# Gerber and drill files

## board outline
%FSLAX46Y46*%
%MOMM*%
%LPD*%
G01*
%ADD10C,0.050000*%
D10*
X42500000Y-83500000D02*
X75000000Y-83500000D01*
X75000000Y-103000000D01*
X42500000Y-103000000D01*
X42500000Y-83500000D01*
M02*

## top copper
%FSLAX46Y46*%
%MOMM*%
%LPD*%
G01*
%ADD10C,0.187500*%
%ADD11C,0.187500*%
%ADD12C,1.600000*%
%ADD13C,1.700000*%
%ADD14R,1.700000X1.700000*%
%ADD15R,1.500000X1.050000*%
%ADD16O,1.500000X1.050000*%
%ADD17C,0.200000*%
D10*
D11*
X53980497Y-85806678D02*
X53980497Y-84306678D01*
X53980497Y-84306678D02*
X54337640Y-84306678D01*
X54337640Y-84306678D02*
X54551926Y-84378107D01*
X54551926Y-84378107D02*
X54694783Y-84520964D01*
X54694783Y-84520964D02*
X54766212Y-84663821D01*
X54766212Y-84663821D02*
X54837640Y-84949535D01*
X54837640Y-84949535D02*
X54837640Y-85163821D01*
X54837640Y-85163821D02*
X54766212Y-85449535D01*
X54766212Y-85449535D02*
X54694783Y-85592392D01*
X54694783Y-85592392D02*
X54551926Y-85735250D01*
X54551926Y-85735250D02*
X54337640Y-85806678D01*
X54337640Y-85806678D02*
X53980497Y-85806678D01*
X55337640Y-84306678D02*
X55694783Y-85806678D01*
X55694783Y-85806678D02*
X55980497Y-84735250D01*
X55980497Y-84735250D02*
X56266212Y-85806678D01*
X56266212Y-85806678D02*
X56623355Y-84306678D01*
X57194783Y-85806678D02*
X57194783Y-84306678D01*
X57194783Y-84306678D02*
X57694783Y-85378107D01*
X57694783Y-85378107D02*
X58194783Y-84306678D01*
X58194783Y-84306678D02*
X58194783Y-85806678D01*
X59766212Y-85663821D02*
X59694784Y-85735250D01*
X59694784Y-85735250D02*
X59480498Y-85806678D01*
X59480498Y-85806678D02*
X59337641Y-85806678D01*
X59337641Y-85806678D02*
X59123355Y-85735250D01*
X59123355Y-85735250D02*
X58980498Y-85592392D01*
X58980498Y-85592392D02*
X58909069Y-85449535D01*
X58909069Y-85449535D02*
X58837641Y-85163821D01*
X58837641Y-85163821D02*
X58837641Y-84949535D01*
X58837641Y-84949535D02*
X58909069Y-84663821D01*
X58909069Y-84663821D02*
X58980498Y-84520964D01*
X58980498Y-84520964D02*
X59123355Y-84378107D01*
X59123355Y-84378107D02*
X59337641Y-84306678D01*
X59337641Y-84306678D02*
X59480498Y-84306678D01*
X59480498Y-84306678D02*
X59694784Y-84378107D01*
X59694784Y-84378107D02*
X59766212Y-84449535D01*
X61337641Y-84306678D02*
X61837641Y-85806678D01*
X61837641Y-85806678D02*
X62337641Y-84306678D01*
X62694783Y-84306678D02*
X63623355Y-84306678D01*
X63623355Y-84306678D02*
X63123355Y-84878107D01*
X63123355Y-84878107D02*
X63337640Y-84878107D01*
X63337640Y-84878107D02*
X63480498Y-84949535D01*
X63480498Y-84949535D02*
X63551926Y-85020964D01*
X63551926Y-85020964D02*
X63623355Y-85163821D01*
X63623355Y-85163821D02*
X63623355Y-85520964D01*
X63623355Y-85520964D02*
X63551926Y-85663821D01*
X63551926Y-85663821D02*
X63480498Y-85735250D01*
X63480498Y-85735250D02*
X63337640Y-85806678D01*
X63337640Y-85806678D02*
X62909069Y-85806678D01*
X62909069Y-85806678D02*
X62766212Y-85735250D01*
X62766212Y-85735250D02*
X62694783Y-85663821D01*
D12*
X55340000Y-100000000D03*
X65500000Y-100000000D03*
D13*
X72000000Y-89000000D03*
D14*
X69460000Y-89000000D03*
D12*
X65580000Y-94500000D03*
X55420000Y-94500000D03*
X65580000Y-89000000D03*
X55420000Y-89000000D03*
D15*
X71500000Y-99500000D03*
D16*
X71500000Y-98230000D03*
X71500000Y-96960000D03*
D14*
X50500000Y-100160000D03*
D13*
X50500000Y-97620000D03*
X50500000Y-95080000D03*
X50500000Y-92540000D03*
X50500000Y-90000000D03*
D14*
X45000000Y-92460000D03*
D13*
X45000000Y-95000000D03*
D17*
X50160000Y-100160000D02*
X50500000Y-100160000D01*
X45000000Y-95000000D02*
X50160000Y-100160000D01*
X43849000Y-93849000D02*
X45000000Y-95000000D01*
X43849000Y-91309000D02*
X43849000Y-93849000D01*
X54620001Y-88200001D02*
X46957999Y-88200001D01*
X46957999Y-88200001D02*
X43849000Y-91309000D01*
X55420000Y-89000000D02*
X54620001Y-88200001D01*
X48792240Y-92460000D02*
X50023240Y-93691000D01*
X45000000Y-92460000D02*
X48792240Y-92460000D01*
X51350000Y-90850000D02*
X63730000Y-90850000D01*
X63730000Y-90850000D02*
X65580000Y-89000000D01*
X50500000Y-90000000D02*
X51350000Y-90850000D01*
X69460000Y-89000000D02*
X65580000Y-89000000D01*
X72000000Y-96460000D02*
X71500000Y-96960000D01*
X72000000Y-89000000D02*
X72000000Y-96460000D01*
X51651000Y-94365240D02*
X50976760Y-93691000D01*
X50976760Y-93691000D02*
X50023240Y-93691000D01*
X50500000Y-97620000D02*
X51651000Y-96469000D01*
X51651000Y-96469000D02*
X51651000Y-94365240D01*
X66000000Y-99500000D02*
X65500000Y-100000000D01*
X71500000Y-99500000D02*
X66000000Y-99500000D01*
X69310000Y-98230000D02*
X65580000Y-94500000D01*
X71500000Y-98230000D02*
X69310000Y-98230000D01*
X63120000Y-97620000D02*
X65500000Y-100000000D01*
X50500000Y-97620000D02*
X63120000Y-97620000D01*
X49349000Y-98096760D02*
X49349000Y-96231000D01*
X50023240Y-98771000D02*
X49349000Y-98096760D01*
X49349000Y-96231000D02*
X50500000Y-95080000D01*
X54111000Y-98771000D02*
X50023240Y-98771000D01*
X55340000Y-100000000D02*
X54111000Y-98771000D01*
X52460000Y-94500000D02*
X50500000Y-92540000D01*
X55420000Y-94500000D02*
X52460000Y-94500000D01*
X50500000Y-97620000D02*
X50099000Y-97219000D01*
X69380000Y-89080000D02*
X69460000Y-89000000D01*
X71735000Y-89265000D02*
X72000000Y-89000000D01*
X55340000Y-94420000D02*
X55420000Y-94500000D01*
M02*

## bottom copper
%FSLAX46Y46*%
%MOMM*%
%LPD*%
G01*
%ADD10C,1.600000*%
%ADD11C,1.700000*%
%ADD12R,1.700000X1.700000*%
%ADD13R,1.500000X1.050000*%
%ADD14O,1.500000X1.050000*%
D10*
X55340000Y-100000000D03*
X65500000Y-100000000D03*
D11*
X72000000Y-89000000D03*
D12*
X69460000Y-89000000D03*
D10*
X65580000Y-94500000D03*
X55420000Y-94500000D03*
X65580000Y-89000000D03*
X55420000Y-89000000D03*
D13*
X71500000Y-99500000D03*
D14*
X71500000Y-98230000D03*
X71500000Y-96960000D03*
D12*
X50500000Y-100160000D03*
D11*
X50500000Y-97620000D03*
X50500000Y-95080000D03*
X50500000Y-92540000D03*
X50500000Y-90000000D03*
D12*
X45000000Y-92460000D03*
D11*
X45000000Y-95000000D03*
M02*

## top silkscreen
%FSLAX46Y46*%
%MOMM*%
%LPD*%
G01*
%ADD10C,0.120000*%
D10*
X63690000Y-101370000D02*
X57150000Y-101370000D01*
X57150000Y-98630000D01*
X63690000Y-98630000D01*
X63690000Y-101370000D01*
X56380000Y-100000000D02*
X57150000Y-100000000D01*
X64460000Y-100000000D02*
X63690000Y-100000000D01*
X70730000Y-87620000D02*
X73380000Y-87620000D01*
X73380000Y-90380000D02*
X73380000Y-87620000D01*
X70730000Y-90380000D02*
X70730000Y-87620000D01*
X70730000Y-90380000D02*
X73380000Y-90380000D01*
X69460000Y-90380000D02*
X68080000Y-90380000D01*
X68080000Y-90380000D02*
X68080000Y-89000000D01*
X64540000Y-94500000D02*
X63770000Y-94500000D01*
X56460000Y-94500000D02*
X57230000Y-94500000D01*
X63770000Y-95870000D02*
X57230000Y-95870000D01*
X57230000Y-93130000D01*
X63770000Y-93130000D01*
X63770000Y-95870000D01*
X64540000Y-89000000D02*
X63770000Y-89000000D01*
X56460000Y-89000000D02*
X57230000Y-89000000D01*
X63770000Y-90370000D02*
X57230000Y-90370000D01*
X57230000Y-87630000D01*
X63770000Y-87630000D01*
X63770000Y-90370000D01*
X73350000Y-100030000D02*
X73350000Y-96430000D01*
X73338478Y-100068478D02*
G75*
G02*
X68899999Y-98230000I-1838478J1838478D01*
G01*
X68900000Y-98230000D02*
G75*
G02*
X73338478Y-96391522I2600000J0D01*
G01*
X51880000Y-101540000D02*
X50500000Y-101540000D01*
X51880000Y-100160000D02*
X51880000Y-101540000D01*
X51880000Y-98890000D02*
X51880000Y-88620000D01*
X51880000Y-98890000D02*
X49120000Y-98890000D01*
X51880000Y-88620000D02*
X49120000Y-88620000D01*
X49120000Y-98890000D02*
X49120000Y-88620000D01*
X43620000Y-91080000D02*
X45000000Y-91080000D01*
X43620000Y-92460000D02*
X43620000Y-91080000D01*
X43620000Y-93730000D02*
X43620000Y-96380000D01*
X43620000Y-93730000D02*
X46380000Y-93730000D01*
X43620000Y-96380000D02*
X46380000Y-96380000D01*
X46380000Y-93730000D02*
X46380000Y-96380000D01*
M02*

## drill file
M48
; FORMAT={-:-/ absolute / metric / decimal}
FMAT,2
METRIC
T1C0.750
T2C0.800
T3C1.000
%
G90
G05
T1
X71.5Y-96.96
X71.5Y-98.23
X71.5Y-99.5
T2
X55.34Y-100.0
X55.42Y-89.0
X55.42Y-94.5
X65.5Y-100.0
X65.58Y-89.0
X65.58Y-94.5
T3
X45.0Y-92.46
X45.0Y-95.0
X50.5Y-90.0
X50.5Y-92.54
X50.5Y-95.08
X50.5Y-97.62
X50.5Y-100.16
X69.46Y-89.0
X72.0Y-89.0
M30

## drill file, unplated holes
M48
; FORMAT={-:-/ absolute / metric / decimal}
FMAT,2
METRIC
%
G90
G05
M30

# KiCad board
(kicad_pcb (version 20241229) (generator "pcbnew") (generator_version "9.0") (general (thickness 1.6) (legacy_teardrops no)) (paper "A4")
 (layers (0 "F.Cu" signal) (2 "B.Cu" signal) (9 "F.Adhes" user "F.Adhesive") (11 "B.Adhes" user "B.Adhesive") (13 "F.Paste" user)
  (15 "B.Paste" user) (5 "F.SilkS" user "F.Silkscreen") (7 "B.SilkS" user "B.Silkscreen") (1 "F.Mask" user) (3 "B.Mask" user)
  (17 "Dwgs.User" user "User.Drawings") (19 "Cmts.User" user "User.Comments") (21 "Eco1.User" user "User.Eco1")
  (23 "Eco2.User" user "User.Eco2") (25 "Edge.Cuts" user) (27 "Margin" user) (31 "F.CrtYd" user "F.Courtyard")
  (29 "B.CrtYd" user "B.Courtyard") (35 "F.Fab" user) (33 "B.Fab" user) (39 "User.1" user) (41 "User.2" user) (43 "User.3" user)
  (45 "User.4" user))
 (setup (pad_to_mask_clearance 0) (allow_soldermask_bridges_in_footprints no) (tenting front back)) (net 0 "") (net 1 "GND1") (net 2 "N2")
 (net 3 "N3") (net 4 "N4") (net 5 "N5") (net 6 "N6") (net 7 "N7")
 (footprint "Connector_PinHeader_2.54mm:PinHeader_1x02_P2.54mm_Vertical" (layer "F.Cu") (at 45 92.46)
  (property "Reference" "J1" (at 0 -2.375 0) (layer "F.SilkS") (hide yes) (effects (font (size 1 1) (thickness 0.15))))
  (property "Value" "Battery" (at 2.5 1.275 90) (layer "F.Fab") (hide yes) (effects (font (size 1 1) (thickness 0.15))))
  (fp_line (start -1.38 -1.38) (end 0 -1.38) (stroke (width 0.12) (type solid)) (layer "F.SilkS"))
  (fp_line (start -1.38 0) (end -1.38 -1.38) (stroke (width 0.12) (type solid)) (layer "F.SilkS"))
  (fp_line (start -1.38 1.27) (end -1.38 3.92) (stroke (width 0.12) (type solid)) (layer "F.SilkS"))
  (fp_line (start -1.38 1.27) (end 1.38 1.27) (stroke (width 0.12) (type solid)) (layer "F.SilkS"))
  (fp_line (start -1.38 3.92) (end 1.38 3.92) (stroke (width 0.12) (type solid)) (layer "F.SilkS"))
  (fp_line (start 1.38 1.27) (end 1.38 3.92) (stroke (width 0.12) (type solid)) (layer "F.SilkS"))
  (pad "1" thru_hole rect (at 0 0) (size 1.7 1.7) (drill 1) (layers "*.Cu" "*.Mask") (remove_unused_layers no) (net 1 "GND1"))
  (pad "2" thru_hole circle (at 0 2.54) (size 1.7 1.7) (drill 1) (layers "*.Cu" "*.Mask") (remove_unused_layers no) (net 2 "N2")))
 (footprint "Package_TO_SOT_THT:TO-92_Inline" (layer "F.Cu") (at 71.5 99.5 90)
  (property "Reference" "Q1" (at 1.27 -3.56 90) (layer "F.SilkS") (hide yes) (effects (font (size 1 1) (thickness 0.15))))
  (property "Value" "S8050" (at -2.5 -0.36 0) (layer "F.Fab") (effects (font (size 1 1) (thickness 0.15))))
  (fp_line (start -0.53 1.85) (end 3.07 1.85) (stroke (width 0.12) (type solid)) (layer "F.SilkS"))
  (fp_arc (start 1.27 -2.6) (mid 3.672087 -0.994977) (end 3.108478 1.838478) (stroke (width 0.12) (type solid)) (layer "F.SilkS"))
  (fp_arc (start -0.568478 1.838478) (mid -1.132087 -0.994977) (end 1.27 -2.6) (stroke (width 0.12) (type solid)) (layer "F.SilkS"))
  (pad "1" thru_hole rect (at 0 0 90) (size 1.05 1.5) (drill 0.75) (layers "*.Cu" "*.Mask") (remove_unused_layers no) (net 1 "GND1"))
  (pad "2" thru_hole oval (at 1.27 0 90) (size 1.05 1.5) (drill 0.75) (layers "*.Cu" "*.Mask") (remove_unused_layers no) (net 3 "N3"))
  (pad "3" thru_hole oval (at 2.54 0 90) (size 1.05 1.5) (drill 0.75) (layers "*.Cu" "*.Mask") (remove_unused_layers no) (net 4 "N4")))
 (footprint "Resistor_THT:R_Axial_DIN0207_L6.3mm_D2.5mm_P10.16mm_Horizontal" (layer "F.Cu") (at 65.58 94.5 180)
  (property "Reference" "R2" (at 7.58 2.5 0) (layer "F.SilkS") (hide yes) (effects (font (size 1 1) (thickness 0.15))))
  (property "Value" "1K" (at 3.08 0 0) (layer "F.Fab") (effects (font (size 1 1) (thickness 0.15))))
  (fp_line (start 9.12 0) (end 8.35 0) (stroke (width 0.12) (type solid)) (layer "F.SilkS"))
  (fp_line (start 1.04 0) (end 1.81 0) (stroke (width 0.12) (type solid)) (layer "F.SilkS"))
  (fp_rect (start 1.81 -1.37) (end 8.35 1.37) (stroke (width 0.12) (type solid)) (fill no) (layer "F.SilkS"))
  (pad "1" thru_hole circle (at 0 0 180) (size 1.6 1.6) (drill 0.8) (layers "*.Cu" "*.Mask") (remove_unused_layers no) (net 3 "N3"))
  (pad "2" thru_hole circle (at 10.16 0 180) (size 1.6 1.6) (drill 0.8) (layers "*.Cu" "*.Mask") (remove_unused_layers no) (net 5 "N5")))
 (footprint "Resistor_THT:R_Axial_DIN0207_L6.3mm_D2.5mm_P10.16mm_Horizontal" (layer "F.Cu") (at 65.5 100 180)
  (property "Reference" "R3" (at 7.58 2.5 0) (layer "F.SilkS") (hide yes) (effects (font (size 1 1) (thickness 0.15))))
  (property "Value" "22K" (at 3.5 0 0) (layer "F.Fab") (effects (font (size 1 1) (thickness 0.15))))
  (fp_line (start 9.12 0) (end 8.35 0) (stroke (width 0.12) (type solid)) (layer "F.SilkS"))
  (fp_line (start 1.04 0) (end 1.81 0) (stroke (width 0.12) (type solid)) (layer "F.SilkS"))
  (fp_rect (start 1.81 -1.37) (end 8.35 1.37) (stroke (width 0.12) (type solid)) (fill no) (layer "F.SilkS"))
  (pad "1" thru_hole circle (at 0 0 180) (size 1.6 1.6) (drill 0.8) (layers "*.Cu" "*.Mask") (remove_unused_layers no) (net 1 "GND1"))
  (pad "2" thru_hole circle (at 10.16 0 180) (size 1.6 1.6) (drill 0.8) (layers "*.Cu" "*.Mask") (remove_unused_layers no) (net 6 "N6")))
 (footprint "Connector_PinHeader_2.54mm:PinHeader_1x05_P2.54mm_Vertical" (layer "F.Cu") (at 50.5 100.16 180)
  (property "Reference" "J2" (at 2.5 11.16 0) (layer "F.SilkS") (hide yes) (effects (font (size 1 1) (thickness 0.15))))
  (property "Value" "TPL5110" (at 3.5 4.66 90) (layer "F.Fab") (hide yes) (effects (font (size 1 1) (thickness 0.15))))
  (fp_line (start 1.38 1.27) (end 1.38 11.54) (stroke (width 0.12) (type solid)) (layer "F.SilkS"))
  (fp_line (start -1.38 11.54) (end 1.38 11.54) (stroke (width 0.12) (type solid)) (layer "F.SilkS"))
  (fp_line (start -1.38 1.27) (end 1.38 1.27) (stroke (width 0.12) (type solid)) (layer "F.SilkS"))
  (fp_line (start -1.38 1.27) (end -1.38 11.54) (stroke (width 0.12) (type solid)) (layer "F.SilkS"))
  (fp_line (start -1.38 0) (end -1.38 -1.38) (stroke (width 0.12) (type solid)) (layer "F.SilkS"))
  (fp_line (start -1.38 -1.38) (end 0 -1.38) (stroke (width 0.12) (type solid)) (layer "F.SilkS"))
  (pad "1" thru_hole rect (at 0 0 180) (size 1.7 1.7) (drill 1) (layers "*.Cu" "*.Mask") (remove_unused_layers no) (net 2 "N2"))
  (pad "2" thru_hole circle (at 0 2.54 180) (size 1.7 1.7) (drill 1) (layers "*.Cu" "*.Mask") (remove_unused_layers no) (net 1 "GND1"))
  (pad "3" thru_hole circle (at 0 5.08 180) (size 1.7 1.7) (drill 1) (layers "*.Cu" "*.Mask") (remove_unused_layers no) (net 6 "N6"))
  (pad "4" thru_hole circle (at 0 7.62 180) (size 1.7 1.7) (drill 1) (layers "*.Cu" "*.Mask") (remove_unused_layers no) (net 5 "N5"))
  (pad "5" thru_hole circle (at 0 10.16 180) (size 1.7 1.7) (drill 1) (layers "*.Cu" "*.Mask") (remove_unused_layers no) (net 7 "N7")))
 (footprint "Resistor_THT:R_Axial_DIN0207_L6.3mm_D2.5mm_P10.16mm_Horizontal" (layer "F.Cu") (at 65.58 89 180)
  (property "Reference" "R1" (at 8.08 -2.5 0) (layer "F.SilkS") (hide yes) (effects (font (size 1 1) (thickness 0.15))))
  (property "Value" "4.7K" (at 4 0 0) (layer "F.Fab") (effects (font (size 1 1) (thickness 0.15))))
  (fp_line (start 9.12 0) (end 8.35 0) (stroke (width 0.12) (type solid)) (layer "F.SilkS"))
  (fp_line (start 1.04 0) (end 1.81 0) (stroke (width 0.12) (type solid)) (layer "F.SilkS"))
  (fp_rect (start 1.81 -1.37) (end 8.35 1.37) (stroke (width 0.12) (type solid)) (fill no) (layer "F.SilkS"))
  (pad "1" thru_hole circle (at 0 0 180) (size 1.6 1.6) (drill 0.8) (layers "*.Cu" "*.Mask") (remove_unused_layers no) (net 7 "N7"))
  (pad "2" thru_hole circle (at 10.16 0 180) (size 1.6 1.6) (drill 0.8) (layers "*.Cu" "*.Mask") (remove_unused_layers no) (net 2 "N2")))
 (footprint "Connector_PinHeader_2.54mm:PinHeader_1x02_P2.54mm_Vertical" (layer "F.Cu") (at 69.46 89 90)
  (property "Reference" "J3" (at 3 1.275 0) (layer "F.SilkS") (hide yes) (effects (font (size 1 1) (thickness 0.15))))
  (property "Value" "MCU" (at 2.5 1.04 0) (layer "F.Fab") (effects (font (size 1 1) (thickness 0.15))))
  (fp_line (start -1.38 -1.38) (end 0 -1.38) (stroke (width 0.12) (type solid)) (layer "F.SilkS"))
  (fp_line (start -1.38 0) (end -1.38 -1.38) (stroke (width 0.12) (type solid)) (layer "F.SilkS"))
  (fp_line (start 1.38 1.27) (end 1.38 3.92) (stroke (width 0.12) (type solid)) (layer "F.SilkS"))
  (fp_line (start -1.38 1.27) (end 1.38 1.27) (stroke (width 0.12) (type solid)) (layer "F.SilkS"))
  (fp_line (start -1.38 1.27) (end -1.38 3.92) (stroke (width 0.12) (type solid)) (layer "F.SilkS"))
  (fp_line (start -1.38 3.92) (end 1.38 3.92) (stroke (width 0.12) (type solid)) (layer "F.SilkS"))
  (pad "1" thru_hole rect (at 0 0 90) (size 1.7 1.7) (drill 1) (layers "*.Cu" "*.Mask") (remove_unused_layers no) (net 7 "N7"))
  (pad "2" thru_hole circle (at 0 2.54 90) (size 1.7 1.7) (drill 1) (layers "*.Cu" "*.Mask") (remove_unused_layers no) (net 4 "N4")))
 (gr_rect (start 42.5 83.5) (end 75 103) (stroke (width 0.05) (type default)) (fill no) (layer "Edge.Cuts"))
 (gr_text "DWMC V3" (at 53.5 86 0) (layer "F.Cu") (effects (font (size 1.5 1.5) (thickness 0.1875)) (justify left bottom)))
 (segment (start 72 89) (end 72 96.46) (width 0.2) (layer "F.Cu") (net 4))
 (segment (start 71.735 89.265) (end 72 89) (width 0.2) (layer "F.Cu") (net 4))
 (segment (start 72 96.46) (end 71.5 96.96) (width 0.2) (layer "F.Cu") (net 4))
 (segment (start 71.5 98.23) (end 69.31 98.23) (width 0.2) (layer "F.Cu") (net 3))
 (segment (start 69.31 98.23) (end 65.58 94.5) (width 0.2) (layer "F.Cu") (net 3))
 (segment (start 43.849 93.849) (end 45 95) (width 0.2) (layer "F.Cu") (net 2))
 (segment (start 45 95) (end 50.16 100.16) (width 0.2) (layer "F.Cu") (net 2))
 (segment (start 43.849 91.309) (end 43.849 93.849) (width 0.2) (layer "F.Cu") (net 2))
 (segment (start 46.957999 88.200001) (end 43.849 91.309) (width 0.2) (layer "F.Cu") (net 2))
 (segment (start 54.620001 88.200001) (end 46.957999 88.200001) (width 0.2) (layer "F.Cu") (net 2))
 (segment (start 55.42 89) (end 54.620001 88.200001) (width 0.2) (layer "F.Cu") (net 2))
 (segment (start 50.16 100.16) (end 50.5 100.16) (width 0.2) (layer "F.Cu") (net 2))
 (segment (start 50.5 90) (end 51.35 90.85) (width 0.2) (layer "F.Cu") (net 7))
 (segment (start 69.38 89.08) (end 69.46 89) (width 0.2) (layer "F.Cu") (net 7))
 (segment (start 69.46 89) (end 65.58 89) (width 0.2) (layer "F.Cu") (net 7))
 (segment (start 51.35 90.85) (end 63.73 90.85) (width 0.2) (layer "F.Cu") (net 7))
 (segment (start 63.73 90.85) (end 65.58 89) (width 0.2) (layer "F.Cu") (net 7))
 (segment (start 49.349 96.231) (end 50.5 95.08) (width 0.2) (layer "F.Cu") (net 6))
 (segment (start 49.349 98.09676) (end 49.349 96.231) (width 0.2) (layer "F.Cu") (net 6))
 (segment (start 55.34 100) (end 54.111 98.771) (width 0.2) (layer "F.Cu") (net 6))
 (segment (start 54.111 98.771) (end 50.02324 98.771) (width 0.2) (layer "F.Cu") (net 6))
 (segment (start 50.02324 98.771) (end 49.349 98.09676) (width 0.2) (layer "F.Cu") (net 6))
 (segment (start 55.42 94.5) (end 52.46 94.5) (width 0.2) (layer "F.Cu") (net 5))
 (segment (start 55.34 94.42) (end 55.42 94.5) (width 0.2) (layer "F.Cu") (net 5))
 (segment (start 52.46 94.5) (end 50.5 92.54) (width 0.2) (layer "F.Cu") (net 5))
 (segment (start 48.79224 92.46) (end 50.02324 93.691) (width 0.2) (layer "F.Cu") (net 1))
 (segment (start 50.5 97.62) (end 51.651 96.469) (width 0.2) (layer "F.Cu") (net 1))
 (segment (start 63.12 97.62) (end 65.5 100) (width 0.2) (layer "F.Cu") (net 1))
 (segment (start 45 92.46) (end 48.79224 92.46) (width 0.2) (layer "F.Cu") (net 1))
 (segment (start 51.651 96.469) (end 51.651 94.36524) (width 0.2) (layer "F.Cu") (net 1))
 (segment (start 51.651 94.36524) (end 50.97676 93.691) (width 0.2) (layer "F.Cu") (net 1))
 (segment (start 50.97676 93.691) (end 50.02324 93.691) (width 0.2) (layer "F.Cu") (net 1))
 (segment (start 71.5 99.5) (end 66 99.5) (width 0.2) (layer "F.Cu") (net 1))
 (segment (start 50.5 97.62) (end 50.099 97.219) (width 0.2) (layer "F.Cu") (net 1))
 (segment (start 50.5 97.62) (end 63.12 97.62) (width 0.2) (layer "F.Cu") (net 1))
 (segment (start 66 99.5) (end 65.5 100) (width 0.2) (layer "F.Cu") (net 1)))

